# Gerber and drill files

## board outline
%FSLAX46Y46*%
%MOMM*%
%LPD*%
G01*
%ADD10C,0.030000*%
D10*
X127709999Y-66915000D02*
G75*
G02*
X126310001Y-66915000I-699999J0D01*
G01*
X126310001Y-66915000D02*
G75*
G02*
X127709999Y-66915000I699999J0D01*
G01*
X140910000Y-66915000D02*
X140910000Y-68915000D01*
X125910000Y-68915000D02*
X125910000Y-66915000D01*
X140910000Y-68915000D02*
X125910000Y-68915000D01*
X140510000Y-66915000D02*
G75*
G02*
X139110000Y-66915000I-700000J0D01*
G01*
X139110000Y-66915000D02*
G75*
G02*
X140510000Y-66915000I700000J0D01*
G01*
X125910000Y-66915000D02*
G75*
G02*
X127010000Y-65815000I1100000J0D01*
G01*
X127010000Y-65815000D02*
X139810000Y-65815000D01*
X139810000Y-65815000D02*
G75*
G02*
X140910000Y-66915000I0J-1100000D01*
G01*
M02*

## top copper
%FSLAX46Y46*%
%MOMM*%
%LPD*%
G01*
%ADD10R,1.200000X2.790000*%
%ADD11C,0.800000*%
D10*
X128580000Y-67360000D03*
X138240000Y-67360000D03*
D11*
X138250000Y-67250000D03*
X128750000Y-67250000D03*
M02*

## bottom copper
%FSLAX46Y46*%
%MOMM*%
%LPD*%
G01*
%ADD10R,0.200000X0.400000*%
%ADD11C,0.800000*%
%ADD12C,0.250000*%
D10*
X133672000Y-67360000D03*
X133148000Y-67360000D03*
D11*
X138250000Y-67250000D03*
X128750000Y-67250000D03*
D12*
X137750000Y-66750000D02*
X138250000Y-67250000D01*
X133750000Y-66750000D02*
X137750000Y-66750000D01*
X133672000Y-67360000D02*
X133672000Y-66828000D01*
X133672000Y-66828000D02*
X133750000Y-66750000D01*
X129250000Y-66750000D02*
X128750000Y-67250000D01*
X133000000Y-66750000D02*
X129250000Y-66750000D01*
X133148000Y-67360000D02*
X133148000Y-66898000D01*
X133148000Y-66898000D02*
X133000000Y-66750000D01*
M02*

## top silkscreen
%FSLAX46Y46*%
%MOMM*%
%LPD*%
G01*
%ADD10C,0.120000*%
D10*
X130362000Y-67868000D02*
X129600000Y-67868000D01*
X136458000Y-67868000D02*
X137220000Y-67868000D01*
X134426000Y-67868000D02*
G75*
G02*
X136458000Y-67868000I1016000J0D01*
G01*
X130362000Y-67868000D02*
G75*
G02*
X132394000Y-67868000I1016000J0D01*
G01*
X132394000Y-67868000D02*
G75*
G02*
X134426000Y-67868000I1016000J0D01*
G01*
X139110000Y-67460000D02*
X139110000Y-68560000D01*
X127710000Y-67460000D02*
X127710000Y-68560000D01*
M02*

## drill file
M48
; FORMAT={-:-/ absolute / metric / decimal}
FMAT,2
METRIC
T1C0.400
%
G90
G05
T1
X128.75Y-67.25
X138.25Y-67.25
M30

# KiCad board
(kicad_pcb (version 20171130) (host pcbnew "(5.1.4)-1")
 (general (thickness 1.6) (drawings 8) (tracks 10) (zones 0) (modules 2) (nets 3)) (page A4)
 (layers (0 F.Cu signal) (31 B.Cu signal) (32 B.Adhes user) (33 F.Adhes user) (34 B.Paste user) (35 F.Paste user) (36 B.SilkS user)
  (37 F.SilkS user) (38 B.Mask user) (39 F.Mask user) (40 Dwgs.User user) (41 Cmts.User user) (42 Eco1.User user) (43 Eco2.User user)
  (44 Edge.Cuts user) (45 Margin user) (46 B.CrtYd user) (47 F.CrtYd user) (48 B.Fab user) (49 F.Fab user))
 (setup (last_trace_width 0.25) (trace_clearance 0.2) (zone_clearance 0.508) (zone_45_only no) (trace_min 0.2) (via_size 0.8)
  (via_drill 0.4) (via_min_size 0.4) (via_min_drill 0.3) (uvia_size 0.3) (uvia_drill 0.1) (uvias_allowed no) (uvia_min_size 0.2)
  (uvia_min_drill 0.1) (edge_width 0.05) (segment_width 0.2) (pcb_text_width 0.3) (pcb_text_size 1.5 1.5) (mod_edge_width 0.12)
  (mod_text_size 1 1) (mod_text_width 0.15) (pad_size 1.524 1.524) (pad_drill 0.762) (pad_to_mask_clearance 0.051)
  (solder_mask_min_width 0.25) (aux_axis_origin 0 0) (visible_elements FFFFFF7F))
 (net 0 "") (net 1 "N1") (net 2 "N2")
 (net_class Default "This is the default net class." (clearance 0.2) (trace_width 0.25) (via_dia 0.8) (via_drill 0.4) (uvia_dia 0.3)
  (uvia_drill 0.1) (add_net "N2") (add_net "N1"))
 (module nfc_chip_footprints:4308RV (layer F.Cu) (at 133.41 67.36)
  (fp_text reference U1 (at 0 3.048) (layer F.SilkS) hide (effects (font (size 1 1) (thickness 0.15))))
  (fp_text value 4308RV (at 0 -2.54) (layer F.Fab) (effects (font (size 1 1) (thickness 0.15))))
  (fp_line (start -3.048 0.508) (end -3.81 0.508) (layer F.SilkS) (width 0.12))
  (fp_line (start 3.048 0.508) (end 3.81 0.508) (layer F.SilkS) (width 0.12))
  (fp_arc (start 2.032 0.508) (end 3.048 0.508) (angle -180) (layer F.SilkS) (width 0.12))
  (fp_arc (start -2.032 0.508) (end -1.016 0.508) (angle -180) (layer F.SilkS) (width 0.12))
  (fp_arc (start 0 0.508) (end 1.016 0.508) (angle -180) (layer F.SilkS) (width 0.12))
  (fp_line (start 5.7 0.1) (end 5.7 1.2) (layer F.SilkS) (width 0.12))
  (fp_line (start -5.7 0.1) (end -5.7 1.2) (layer F.SilkS) (width 0.12))
  (pad A2 smd rect (at -4.23 0 180) (size 1.2 2.79) (drill (offset 0.6 0)) (layers F.Cu F.Paste F.Mask) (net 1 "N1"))
  (pad A1 smd rect (at 4.23 0) (size 1.2 2.79) (drill (offset 0.6 0)) (layers F.Cu F.Paste F.Mask) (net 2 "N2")))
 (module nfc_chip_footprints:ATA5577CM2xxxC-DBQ (layer B.Cu) (at 133.41 67.36)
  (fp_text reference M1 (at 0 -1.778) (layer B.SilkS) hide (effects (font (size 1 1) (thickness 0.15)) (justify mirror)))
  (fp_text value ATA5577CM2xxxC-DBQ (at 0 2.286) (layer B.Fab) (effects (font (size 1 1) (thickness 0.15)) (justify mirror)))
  (pad C1 smd rect (at 0.262 0) (size 0.2 0.4) (layers B.Cu B.Paste B.Mask) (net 2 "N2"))
  (pad C2 smd rect (at -0.262 0) (size 0.2 0.4) (layers B.Cu B.Paste B.Mask) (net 1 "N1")))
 (gr_circle (center 127.01 66.915) (end 127.709999 66.915) (layer Edge.Cuts) (width 0.03))
 (gr_line (start 140.91 66.915) (end 140.91 68.915) (layer Edge.Cuts) (width 0.03))
 (gr_line (start 125.91 68.915) (end 125.91 66.915) (layer Edge.Cuts) (width 0.03))
 (gr_line (start 140.91 68.915) (end 125.91 68.915) (layer Edge.Cuts) (width 0.03))
 (gr_circle (center 139.81 66.915) (end 140.51 66.915) (layer Edge.Cuts) (width 0.03))
 (gr_arc (start 127.01 66.915) (end 127.01 65.815) (angle -90) (layer Edge.Cuts) (width 0.03))
 (gr_line (start 127.01 65.815) (end 139.81 65.815) (layer Edge.Cuts) (width 0.03))
 (gr_arc (start 139.81 66.915) (end 140.91 66.915) (angle -90) (layer Edge.Cuts) (width 0.03))
 (via (at 138.25 67.25) (size 0.8) (drill 0.4) (layers F.Cu B.Cu) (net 2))
 (segment (start 137.75 66.75) (end 138.25 67.25) (width 0.25) (layer B.Cu) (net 2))
 (segment (start 133.75 66.75) (end 137.75 66.75) (width 0.25) (layer B.Cu) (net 2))
 (segment (start 133.672 67.36) (end 133.672 66.828) (width 0.25) (layer B.Cu) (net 2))
 (segment (start 133.672 66.828) (end 133.75 66.75) (width 0.25) (layer B.Cu) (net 2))
 (via (at 128.75 67.25) (size 0.8) (drill 0.4) (layers F.Cu B.Cu) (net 1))
 (segment (start 129.25 66.75) (end 128.75 67.25) (width 0.25) (layer B.Cu) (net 1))
 (segment (start 133 66.75) (end 129.25 66.75) (width 0.25) (layer B.Cu) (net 1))
 (segment (start 133.148 67.36) (end 133.148 66.898) (width 0.25) (layer B.Cu) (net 1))
 (segment (start 133.148 66.898) (end 133 66.75) (width 0.25) (layer B.Cu) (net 1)))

